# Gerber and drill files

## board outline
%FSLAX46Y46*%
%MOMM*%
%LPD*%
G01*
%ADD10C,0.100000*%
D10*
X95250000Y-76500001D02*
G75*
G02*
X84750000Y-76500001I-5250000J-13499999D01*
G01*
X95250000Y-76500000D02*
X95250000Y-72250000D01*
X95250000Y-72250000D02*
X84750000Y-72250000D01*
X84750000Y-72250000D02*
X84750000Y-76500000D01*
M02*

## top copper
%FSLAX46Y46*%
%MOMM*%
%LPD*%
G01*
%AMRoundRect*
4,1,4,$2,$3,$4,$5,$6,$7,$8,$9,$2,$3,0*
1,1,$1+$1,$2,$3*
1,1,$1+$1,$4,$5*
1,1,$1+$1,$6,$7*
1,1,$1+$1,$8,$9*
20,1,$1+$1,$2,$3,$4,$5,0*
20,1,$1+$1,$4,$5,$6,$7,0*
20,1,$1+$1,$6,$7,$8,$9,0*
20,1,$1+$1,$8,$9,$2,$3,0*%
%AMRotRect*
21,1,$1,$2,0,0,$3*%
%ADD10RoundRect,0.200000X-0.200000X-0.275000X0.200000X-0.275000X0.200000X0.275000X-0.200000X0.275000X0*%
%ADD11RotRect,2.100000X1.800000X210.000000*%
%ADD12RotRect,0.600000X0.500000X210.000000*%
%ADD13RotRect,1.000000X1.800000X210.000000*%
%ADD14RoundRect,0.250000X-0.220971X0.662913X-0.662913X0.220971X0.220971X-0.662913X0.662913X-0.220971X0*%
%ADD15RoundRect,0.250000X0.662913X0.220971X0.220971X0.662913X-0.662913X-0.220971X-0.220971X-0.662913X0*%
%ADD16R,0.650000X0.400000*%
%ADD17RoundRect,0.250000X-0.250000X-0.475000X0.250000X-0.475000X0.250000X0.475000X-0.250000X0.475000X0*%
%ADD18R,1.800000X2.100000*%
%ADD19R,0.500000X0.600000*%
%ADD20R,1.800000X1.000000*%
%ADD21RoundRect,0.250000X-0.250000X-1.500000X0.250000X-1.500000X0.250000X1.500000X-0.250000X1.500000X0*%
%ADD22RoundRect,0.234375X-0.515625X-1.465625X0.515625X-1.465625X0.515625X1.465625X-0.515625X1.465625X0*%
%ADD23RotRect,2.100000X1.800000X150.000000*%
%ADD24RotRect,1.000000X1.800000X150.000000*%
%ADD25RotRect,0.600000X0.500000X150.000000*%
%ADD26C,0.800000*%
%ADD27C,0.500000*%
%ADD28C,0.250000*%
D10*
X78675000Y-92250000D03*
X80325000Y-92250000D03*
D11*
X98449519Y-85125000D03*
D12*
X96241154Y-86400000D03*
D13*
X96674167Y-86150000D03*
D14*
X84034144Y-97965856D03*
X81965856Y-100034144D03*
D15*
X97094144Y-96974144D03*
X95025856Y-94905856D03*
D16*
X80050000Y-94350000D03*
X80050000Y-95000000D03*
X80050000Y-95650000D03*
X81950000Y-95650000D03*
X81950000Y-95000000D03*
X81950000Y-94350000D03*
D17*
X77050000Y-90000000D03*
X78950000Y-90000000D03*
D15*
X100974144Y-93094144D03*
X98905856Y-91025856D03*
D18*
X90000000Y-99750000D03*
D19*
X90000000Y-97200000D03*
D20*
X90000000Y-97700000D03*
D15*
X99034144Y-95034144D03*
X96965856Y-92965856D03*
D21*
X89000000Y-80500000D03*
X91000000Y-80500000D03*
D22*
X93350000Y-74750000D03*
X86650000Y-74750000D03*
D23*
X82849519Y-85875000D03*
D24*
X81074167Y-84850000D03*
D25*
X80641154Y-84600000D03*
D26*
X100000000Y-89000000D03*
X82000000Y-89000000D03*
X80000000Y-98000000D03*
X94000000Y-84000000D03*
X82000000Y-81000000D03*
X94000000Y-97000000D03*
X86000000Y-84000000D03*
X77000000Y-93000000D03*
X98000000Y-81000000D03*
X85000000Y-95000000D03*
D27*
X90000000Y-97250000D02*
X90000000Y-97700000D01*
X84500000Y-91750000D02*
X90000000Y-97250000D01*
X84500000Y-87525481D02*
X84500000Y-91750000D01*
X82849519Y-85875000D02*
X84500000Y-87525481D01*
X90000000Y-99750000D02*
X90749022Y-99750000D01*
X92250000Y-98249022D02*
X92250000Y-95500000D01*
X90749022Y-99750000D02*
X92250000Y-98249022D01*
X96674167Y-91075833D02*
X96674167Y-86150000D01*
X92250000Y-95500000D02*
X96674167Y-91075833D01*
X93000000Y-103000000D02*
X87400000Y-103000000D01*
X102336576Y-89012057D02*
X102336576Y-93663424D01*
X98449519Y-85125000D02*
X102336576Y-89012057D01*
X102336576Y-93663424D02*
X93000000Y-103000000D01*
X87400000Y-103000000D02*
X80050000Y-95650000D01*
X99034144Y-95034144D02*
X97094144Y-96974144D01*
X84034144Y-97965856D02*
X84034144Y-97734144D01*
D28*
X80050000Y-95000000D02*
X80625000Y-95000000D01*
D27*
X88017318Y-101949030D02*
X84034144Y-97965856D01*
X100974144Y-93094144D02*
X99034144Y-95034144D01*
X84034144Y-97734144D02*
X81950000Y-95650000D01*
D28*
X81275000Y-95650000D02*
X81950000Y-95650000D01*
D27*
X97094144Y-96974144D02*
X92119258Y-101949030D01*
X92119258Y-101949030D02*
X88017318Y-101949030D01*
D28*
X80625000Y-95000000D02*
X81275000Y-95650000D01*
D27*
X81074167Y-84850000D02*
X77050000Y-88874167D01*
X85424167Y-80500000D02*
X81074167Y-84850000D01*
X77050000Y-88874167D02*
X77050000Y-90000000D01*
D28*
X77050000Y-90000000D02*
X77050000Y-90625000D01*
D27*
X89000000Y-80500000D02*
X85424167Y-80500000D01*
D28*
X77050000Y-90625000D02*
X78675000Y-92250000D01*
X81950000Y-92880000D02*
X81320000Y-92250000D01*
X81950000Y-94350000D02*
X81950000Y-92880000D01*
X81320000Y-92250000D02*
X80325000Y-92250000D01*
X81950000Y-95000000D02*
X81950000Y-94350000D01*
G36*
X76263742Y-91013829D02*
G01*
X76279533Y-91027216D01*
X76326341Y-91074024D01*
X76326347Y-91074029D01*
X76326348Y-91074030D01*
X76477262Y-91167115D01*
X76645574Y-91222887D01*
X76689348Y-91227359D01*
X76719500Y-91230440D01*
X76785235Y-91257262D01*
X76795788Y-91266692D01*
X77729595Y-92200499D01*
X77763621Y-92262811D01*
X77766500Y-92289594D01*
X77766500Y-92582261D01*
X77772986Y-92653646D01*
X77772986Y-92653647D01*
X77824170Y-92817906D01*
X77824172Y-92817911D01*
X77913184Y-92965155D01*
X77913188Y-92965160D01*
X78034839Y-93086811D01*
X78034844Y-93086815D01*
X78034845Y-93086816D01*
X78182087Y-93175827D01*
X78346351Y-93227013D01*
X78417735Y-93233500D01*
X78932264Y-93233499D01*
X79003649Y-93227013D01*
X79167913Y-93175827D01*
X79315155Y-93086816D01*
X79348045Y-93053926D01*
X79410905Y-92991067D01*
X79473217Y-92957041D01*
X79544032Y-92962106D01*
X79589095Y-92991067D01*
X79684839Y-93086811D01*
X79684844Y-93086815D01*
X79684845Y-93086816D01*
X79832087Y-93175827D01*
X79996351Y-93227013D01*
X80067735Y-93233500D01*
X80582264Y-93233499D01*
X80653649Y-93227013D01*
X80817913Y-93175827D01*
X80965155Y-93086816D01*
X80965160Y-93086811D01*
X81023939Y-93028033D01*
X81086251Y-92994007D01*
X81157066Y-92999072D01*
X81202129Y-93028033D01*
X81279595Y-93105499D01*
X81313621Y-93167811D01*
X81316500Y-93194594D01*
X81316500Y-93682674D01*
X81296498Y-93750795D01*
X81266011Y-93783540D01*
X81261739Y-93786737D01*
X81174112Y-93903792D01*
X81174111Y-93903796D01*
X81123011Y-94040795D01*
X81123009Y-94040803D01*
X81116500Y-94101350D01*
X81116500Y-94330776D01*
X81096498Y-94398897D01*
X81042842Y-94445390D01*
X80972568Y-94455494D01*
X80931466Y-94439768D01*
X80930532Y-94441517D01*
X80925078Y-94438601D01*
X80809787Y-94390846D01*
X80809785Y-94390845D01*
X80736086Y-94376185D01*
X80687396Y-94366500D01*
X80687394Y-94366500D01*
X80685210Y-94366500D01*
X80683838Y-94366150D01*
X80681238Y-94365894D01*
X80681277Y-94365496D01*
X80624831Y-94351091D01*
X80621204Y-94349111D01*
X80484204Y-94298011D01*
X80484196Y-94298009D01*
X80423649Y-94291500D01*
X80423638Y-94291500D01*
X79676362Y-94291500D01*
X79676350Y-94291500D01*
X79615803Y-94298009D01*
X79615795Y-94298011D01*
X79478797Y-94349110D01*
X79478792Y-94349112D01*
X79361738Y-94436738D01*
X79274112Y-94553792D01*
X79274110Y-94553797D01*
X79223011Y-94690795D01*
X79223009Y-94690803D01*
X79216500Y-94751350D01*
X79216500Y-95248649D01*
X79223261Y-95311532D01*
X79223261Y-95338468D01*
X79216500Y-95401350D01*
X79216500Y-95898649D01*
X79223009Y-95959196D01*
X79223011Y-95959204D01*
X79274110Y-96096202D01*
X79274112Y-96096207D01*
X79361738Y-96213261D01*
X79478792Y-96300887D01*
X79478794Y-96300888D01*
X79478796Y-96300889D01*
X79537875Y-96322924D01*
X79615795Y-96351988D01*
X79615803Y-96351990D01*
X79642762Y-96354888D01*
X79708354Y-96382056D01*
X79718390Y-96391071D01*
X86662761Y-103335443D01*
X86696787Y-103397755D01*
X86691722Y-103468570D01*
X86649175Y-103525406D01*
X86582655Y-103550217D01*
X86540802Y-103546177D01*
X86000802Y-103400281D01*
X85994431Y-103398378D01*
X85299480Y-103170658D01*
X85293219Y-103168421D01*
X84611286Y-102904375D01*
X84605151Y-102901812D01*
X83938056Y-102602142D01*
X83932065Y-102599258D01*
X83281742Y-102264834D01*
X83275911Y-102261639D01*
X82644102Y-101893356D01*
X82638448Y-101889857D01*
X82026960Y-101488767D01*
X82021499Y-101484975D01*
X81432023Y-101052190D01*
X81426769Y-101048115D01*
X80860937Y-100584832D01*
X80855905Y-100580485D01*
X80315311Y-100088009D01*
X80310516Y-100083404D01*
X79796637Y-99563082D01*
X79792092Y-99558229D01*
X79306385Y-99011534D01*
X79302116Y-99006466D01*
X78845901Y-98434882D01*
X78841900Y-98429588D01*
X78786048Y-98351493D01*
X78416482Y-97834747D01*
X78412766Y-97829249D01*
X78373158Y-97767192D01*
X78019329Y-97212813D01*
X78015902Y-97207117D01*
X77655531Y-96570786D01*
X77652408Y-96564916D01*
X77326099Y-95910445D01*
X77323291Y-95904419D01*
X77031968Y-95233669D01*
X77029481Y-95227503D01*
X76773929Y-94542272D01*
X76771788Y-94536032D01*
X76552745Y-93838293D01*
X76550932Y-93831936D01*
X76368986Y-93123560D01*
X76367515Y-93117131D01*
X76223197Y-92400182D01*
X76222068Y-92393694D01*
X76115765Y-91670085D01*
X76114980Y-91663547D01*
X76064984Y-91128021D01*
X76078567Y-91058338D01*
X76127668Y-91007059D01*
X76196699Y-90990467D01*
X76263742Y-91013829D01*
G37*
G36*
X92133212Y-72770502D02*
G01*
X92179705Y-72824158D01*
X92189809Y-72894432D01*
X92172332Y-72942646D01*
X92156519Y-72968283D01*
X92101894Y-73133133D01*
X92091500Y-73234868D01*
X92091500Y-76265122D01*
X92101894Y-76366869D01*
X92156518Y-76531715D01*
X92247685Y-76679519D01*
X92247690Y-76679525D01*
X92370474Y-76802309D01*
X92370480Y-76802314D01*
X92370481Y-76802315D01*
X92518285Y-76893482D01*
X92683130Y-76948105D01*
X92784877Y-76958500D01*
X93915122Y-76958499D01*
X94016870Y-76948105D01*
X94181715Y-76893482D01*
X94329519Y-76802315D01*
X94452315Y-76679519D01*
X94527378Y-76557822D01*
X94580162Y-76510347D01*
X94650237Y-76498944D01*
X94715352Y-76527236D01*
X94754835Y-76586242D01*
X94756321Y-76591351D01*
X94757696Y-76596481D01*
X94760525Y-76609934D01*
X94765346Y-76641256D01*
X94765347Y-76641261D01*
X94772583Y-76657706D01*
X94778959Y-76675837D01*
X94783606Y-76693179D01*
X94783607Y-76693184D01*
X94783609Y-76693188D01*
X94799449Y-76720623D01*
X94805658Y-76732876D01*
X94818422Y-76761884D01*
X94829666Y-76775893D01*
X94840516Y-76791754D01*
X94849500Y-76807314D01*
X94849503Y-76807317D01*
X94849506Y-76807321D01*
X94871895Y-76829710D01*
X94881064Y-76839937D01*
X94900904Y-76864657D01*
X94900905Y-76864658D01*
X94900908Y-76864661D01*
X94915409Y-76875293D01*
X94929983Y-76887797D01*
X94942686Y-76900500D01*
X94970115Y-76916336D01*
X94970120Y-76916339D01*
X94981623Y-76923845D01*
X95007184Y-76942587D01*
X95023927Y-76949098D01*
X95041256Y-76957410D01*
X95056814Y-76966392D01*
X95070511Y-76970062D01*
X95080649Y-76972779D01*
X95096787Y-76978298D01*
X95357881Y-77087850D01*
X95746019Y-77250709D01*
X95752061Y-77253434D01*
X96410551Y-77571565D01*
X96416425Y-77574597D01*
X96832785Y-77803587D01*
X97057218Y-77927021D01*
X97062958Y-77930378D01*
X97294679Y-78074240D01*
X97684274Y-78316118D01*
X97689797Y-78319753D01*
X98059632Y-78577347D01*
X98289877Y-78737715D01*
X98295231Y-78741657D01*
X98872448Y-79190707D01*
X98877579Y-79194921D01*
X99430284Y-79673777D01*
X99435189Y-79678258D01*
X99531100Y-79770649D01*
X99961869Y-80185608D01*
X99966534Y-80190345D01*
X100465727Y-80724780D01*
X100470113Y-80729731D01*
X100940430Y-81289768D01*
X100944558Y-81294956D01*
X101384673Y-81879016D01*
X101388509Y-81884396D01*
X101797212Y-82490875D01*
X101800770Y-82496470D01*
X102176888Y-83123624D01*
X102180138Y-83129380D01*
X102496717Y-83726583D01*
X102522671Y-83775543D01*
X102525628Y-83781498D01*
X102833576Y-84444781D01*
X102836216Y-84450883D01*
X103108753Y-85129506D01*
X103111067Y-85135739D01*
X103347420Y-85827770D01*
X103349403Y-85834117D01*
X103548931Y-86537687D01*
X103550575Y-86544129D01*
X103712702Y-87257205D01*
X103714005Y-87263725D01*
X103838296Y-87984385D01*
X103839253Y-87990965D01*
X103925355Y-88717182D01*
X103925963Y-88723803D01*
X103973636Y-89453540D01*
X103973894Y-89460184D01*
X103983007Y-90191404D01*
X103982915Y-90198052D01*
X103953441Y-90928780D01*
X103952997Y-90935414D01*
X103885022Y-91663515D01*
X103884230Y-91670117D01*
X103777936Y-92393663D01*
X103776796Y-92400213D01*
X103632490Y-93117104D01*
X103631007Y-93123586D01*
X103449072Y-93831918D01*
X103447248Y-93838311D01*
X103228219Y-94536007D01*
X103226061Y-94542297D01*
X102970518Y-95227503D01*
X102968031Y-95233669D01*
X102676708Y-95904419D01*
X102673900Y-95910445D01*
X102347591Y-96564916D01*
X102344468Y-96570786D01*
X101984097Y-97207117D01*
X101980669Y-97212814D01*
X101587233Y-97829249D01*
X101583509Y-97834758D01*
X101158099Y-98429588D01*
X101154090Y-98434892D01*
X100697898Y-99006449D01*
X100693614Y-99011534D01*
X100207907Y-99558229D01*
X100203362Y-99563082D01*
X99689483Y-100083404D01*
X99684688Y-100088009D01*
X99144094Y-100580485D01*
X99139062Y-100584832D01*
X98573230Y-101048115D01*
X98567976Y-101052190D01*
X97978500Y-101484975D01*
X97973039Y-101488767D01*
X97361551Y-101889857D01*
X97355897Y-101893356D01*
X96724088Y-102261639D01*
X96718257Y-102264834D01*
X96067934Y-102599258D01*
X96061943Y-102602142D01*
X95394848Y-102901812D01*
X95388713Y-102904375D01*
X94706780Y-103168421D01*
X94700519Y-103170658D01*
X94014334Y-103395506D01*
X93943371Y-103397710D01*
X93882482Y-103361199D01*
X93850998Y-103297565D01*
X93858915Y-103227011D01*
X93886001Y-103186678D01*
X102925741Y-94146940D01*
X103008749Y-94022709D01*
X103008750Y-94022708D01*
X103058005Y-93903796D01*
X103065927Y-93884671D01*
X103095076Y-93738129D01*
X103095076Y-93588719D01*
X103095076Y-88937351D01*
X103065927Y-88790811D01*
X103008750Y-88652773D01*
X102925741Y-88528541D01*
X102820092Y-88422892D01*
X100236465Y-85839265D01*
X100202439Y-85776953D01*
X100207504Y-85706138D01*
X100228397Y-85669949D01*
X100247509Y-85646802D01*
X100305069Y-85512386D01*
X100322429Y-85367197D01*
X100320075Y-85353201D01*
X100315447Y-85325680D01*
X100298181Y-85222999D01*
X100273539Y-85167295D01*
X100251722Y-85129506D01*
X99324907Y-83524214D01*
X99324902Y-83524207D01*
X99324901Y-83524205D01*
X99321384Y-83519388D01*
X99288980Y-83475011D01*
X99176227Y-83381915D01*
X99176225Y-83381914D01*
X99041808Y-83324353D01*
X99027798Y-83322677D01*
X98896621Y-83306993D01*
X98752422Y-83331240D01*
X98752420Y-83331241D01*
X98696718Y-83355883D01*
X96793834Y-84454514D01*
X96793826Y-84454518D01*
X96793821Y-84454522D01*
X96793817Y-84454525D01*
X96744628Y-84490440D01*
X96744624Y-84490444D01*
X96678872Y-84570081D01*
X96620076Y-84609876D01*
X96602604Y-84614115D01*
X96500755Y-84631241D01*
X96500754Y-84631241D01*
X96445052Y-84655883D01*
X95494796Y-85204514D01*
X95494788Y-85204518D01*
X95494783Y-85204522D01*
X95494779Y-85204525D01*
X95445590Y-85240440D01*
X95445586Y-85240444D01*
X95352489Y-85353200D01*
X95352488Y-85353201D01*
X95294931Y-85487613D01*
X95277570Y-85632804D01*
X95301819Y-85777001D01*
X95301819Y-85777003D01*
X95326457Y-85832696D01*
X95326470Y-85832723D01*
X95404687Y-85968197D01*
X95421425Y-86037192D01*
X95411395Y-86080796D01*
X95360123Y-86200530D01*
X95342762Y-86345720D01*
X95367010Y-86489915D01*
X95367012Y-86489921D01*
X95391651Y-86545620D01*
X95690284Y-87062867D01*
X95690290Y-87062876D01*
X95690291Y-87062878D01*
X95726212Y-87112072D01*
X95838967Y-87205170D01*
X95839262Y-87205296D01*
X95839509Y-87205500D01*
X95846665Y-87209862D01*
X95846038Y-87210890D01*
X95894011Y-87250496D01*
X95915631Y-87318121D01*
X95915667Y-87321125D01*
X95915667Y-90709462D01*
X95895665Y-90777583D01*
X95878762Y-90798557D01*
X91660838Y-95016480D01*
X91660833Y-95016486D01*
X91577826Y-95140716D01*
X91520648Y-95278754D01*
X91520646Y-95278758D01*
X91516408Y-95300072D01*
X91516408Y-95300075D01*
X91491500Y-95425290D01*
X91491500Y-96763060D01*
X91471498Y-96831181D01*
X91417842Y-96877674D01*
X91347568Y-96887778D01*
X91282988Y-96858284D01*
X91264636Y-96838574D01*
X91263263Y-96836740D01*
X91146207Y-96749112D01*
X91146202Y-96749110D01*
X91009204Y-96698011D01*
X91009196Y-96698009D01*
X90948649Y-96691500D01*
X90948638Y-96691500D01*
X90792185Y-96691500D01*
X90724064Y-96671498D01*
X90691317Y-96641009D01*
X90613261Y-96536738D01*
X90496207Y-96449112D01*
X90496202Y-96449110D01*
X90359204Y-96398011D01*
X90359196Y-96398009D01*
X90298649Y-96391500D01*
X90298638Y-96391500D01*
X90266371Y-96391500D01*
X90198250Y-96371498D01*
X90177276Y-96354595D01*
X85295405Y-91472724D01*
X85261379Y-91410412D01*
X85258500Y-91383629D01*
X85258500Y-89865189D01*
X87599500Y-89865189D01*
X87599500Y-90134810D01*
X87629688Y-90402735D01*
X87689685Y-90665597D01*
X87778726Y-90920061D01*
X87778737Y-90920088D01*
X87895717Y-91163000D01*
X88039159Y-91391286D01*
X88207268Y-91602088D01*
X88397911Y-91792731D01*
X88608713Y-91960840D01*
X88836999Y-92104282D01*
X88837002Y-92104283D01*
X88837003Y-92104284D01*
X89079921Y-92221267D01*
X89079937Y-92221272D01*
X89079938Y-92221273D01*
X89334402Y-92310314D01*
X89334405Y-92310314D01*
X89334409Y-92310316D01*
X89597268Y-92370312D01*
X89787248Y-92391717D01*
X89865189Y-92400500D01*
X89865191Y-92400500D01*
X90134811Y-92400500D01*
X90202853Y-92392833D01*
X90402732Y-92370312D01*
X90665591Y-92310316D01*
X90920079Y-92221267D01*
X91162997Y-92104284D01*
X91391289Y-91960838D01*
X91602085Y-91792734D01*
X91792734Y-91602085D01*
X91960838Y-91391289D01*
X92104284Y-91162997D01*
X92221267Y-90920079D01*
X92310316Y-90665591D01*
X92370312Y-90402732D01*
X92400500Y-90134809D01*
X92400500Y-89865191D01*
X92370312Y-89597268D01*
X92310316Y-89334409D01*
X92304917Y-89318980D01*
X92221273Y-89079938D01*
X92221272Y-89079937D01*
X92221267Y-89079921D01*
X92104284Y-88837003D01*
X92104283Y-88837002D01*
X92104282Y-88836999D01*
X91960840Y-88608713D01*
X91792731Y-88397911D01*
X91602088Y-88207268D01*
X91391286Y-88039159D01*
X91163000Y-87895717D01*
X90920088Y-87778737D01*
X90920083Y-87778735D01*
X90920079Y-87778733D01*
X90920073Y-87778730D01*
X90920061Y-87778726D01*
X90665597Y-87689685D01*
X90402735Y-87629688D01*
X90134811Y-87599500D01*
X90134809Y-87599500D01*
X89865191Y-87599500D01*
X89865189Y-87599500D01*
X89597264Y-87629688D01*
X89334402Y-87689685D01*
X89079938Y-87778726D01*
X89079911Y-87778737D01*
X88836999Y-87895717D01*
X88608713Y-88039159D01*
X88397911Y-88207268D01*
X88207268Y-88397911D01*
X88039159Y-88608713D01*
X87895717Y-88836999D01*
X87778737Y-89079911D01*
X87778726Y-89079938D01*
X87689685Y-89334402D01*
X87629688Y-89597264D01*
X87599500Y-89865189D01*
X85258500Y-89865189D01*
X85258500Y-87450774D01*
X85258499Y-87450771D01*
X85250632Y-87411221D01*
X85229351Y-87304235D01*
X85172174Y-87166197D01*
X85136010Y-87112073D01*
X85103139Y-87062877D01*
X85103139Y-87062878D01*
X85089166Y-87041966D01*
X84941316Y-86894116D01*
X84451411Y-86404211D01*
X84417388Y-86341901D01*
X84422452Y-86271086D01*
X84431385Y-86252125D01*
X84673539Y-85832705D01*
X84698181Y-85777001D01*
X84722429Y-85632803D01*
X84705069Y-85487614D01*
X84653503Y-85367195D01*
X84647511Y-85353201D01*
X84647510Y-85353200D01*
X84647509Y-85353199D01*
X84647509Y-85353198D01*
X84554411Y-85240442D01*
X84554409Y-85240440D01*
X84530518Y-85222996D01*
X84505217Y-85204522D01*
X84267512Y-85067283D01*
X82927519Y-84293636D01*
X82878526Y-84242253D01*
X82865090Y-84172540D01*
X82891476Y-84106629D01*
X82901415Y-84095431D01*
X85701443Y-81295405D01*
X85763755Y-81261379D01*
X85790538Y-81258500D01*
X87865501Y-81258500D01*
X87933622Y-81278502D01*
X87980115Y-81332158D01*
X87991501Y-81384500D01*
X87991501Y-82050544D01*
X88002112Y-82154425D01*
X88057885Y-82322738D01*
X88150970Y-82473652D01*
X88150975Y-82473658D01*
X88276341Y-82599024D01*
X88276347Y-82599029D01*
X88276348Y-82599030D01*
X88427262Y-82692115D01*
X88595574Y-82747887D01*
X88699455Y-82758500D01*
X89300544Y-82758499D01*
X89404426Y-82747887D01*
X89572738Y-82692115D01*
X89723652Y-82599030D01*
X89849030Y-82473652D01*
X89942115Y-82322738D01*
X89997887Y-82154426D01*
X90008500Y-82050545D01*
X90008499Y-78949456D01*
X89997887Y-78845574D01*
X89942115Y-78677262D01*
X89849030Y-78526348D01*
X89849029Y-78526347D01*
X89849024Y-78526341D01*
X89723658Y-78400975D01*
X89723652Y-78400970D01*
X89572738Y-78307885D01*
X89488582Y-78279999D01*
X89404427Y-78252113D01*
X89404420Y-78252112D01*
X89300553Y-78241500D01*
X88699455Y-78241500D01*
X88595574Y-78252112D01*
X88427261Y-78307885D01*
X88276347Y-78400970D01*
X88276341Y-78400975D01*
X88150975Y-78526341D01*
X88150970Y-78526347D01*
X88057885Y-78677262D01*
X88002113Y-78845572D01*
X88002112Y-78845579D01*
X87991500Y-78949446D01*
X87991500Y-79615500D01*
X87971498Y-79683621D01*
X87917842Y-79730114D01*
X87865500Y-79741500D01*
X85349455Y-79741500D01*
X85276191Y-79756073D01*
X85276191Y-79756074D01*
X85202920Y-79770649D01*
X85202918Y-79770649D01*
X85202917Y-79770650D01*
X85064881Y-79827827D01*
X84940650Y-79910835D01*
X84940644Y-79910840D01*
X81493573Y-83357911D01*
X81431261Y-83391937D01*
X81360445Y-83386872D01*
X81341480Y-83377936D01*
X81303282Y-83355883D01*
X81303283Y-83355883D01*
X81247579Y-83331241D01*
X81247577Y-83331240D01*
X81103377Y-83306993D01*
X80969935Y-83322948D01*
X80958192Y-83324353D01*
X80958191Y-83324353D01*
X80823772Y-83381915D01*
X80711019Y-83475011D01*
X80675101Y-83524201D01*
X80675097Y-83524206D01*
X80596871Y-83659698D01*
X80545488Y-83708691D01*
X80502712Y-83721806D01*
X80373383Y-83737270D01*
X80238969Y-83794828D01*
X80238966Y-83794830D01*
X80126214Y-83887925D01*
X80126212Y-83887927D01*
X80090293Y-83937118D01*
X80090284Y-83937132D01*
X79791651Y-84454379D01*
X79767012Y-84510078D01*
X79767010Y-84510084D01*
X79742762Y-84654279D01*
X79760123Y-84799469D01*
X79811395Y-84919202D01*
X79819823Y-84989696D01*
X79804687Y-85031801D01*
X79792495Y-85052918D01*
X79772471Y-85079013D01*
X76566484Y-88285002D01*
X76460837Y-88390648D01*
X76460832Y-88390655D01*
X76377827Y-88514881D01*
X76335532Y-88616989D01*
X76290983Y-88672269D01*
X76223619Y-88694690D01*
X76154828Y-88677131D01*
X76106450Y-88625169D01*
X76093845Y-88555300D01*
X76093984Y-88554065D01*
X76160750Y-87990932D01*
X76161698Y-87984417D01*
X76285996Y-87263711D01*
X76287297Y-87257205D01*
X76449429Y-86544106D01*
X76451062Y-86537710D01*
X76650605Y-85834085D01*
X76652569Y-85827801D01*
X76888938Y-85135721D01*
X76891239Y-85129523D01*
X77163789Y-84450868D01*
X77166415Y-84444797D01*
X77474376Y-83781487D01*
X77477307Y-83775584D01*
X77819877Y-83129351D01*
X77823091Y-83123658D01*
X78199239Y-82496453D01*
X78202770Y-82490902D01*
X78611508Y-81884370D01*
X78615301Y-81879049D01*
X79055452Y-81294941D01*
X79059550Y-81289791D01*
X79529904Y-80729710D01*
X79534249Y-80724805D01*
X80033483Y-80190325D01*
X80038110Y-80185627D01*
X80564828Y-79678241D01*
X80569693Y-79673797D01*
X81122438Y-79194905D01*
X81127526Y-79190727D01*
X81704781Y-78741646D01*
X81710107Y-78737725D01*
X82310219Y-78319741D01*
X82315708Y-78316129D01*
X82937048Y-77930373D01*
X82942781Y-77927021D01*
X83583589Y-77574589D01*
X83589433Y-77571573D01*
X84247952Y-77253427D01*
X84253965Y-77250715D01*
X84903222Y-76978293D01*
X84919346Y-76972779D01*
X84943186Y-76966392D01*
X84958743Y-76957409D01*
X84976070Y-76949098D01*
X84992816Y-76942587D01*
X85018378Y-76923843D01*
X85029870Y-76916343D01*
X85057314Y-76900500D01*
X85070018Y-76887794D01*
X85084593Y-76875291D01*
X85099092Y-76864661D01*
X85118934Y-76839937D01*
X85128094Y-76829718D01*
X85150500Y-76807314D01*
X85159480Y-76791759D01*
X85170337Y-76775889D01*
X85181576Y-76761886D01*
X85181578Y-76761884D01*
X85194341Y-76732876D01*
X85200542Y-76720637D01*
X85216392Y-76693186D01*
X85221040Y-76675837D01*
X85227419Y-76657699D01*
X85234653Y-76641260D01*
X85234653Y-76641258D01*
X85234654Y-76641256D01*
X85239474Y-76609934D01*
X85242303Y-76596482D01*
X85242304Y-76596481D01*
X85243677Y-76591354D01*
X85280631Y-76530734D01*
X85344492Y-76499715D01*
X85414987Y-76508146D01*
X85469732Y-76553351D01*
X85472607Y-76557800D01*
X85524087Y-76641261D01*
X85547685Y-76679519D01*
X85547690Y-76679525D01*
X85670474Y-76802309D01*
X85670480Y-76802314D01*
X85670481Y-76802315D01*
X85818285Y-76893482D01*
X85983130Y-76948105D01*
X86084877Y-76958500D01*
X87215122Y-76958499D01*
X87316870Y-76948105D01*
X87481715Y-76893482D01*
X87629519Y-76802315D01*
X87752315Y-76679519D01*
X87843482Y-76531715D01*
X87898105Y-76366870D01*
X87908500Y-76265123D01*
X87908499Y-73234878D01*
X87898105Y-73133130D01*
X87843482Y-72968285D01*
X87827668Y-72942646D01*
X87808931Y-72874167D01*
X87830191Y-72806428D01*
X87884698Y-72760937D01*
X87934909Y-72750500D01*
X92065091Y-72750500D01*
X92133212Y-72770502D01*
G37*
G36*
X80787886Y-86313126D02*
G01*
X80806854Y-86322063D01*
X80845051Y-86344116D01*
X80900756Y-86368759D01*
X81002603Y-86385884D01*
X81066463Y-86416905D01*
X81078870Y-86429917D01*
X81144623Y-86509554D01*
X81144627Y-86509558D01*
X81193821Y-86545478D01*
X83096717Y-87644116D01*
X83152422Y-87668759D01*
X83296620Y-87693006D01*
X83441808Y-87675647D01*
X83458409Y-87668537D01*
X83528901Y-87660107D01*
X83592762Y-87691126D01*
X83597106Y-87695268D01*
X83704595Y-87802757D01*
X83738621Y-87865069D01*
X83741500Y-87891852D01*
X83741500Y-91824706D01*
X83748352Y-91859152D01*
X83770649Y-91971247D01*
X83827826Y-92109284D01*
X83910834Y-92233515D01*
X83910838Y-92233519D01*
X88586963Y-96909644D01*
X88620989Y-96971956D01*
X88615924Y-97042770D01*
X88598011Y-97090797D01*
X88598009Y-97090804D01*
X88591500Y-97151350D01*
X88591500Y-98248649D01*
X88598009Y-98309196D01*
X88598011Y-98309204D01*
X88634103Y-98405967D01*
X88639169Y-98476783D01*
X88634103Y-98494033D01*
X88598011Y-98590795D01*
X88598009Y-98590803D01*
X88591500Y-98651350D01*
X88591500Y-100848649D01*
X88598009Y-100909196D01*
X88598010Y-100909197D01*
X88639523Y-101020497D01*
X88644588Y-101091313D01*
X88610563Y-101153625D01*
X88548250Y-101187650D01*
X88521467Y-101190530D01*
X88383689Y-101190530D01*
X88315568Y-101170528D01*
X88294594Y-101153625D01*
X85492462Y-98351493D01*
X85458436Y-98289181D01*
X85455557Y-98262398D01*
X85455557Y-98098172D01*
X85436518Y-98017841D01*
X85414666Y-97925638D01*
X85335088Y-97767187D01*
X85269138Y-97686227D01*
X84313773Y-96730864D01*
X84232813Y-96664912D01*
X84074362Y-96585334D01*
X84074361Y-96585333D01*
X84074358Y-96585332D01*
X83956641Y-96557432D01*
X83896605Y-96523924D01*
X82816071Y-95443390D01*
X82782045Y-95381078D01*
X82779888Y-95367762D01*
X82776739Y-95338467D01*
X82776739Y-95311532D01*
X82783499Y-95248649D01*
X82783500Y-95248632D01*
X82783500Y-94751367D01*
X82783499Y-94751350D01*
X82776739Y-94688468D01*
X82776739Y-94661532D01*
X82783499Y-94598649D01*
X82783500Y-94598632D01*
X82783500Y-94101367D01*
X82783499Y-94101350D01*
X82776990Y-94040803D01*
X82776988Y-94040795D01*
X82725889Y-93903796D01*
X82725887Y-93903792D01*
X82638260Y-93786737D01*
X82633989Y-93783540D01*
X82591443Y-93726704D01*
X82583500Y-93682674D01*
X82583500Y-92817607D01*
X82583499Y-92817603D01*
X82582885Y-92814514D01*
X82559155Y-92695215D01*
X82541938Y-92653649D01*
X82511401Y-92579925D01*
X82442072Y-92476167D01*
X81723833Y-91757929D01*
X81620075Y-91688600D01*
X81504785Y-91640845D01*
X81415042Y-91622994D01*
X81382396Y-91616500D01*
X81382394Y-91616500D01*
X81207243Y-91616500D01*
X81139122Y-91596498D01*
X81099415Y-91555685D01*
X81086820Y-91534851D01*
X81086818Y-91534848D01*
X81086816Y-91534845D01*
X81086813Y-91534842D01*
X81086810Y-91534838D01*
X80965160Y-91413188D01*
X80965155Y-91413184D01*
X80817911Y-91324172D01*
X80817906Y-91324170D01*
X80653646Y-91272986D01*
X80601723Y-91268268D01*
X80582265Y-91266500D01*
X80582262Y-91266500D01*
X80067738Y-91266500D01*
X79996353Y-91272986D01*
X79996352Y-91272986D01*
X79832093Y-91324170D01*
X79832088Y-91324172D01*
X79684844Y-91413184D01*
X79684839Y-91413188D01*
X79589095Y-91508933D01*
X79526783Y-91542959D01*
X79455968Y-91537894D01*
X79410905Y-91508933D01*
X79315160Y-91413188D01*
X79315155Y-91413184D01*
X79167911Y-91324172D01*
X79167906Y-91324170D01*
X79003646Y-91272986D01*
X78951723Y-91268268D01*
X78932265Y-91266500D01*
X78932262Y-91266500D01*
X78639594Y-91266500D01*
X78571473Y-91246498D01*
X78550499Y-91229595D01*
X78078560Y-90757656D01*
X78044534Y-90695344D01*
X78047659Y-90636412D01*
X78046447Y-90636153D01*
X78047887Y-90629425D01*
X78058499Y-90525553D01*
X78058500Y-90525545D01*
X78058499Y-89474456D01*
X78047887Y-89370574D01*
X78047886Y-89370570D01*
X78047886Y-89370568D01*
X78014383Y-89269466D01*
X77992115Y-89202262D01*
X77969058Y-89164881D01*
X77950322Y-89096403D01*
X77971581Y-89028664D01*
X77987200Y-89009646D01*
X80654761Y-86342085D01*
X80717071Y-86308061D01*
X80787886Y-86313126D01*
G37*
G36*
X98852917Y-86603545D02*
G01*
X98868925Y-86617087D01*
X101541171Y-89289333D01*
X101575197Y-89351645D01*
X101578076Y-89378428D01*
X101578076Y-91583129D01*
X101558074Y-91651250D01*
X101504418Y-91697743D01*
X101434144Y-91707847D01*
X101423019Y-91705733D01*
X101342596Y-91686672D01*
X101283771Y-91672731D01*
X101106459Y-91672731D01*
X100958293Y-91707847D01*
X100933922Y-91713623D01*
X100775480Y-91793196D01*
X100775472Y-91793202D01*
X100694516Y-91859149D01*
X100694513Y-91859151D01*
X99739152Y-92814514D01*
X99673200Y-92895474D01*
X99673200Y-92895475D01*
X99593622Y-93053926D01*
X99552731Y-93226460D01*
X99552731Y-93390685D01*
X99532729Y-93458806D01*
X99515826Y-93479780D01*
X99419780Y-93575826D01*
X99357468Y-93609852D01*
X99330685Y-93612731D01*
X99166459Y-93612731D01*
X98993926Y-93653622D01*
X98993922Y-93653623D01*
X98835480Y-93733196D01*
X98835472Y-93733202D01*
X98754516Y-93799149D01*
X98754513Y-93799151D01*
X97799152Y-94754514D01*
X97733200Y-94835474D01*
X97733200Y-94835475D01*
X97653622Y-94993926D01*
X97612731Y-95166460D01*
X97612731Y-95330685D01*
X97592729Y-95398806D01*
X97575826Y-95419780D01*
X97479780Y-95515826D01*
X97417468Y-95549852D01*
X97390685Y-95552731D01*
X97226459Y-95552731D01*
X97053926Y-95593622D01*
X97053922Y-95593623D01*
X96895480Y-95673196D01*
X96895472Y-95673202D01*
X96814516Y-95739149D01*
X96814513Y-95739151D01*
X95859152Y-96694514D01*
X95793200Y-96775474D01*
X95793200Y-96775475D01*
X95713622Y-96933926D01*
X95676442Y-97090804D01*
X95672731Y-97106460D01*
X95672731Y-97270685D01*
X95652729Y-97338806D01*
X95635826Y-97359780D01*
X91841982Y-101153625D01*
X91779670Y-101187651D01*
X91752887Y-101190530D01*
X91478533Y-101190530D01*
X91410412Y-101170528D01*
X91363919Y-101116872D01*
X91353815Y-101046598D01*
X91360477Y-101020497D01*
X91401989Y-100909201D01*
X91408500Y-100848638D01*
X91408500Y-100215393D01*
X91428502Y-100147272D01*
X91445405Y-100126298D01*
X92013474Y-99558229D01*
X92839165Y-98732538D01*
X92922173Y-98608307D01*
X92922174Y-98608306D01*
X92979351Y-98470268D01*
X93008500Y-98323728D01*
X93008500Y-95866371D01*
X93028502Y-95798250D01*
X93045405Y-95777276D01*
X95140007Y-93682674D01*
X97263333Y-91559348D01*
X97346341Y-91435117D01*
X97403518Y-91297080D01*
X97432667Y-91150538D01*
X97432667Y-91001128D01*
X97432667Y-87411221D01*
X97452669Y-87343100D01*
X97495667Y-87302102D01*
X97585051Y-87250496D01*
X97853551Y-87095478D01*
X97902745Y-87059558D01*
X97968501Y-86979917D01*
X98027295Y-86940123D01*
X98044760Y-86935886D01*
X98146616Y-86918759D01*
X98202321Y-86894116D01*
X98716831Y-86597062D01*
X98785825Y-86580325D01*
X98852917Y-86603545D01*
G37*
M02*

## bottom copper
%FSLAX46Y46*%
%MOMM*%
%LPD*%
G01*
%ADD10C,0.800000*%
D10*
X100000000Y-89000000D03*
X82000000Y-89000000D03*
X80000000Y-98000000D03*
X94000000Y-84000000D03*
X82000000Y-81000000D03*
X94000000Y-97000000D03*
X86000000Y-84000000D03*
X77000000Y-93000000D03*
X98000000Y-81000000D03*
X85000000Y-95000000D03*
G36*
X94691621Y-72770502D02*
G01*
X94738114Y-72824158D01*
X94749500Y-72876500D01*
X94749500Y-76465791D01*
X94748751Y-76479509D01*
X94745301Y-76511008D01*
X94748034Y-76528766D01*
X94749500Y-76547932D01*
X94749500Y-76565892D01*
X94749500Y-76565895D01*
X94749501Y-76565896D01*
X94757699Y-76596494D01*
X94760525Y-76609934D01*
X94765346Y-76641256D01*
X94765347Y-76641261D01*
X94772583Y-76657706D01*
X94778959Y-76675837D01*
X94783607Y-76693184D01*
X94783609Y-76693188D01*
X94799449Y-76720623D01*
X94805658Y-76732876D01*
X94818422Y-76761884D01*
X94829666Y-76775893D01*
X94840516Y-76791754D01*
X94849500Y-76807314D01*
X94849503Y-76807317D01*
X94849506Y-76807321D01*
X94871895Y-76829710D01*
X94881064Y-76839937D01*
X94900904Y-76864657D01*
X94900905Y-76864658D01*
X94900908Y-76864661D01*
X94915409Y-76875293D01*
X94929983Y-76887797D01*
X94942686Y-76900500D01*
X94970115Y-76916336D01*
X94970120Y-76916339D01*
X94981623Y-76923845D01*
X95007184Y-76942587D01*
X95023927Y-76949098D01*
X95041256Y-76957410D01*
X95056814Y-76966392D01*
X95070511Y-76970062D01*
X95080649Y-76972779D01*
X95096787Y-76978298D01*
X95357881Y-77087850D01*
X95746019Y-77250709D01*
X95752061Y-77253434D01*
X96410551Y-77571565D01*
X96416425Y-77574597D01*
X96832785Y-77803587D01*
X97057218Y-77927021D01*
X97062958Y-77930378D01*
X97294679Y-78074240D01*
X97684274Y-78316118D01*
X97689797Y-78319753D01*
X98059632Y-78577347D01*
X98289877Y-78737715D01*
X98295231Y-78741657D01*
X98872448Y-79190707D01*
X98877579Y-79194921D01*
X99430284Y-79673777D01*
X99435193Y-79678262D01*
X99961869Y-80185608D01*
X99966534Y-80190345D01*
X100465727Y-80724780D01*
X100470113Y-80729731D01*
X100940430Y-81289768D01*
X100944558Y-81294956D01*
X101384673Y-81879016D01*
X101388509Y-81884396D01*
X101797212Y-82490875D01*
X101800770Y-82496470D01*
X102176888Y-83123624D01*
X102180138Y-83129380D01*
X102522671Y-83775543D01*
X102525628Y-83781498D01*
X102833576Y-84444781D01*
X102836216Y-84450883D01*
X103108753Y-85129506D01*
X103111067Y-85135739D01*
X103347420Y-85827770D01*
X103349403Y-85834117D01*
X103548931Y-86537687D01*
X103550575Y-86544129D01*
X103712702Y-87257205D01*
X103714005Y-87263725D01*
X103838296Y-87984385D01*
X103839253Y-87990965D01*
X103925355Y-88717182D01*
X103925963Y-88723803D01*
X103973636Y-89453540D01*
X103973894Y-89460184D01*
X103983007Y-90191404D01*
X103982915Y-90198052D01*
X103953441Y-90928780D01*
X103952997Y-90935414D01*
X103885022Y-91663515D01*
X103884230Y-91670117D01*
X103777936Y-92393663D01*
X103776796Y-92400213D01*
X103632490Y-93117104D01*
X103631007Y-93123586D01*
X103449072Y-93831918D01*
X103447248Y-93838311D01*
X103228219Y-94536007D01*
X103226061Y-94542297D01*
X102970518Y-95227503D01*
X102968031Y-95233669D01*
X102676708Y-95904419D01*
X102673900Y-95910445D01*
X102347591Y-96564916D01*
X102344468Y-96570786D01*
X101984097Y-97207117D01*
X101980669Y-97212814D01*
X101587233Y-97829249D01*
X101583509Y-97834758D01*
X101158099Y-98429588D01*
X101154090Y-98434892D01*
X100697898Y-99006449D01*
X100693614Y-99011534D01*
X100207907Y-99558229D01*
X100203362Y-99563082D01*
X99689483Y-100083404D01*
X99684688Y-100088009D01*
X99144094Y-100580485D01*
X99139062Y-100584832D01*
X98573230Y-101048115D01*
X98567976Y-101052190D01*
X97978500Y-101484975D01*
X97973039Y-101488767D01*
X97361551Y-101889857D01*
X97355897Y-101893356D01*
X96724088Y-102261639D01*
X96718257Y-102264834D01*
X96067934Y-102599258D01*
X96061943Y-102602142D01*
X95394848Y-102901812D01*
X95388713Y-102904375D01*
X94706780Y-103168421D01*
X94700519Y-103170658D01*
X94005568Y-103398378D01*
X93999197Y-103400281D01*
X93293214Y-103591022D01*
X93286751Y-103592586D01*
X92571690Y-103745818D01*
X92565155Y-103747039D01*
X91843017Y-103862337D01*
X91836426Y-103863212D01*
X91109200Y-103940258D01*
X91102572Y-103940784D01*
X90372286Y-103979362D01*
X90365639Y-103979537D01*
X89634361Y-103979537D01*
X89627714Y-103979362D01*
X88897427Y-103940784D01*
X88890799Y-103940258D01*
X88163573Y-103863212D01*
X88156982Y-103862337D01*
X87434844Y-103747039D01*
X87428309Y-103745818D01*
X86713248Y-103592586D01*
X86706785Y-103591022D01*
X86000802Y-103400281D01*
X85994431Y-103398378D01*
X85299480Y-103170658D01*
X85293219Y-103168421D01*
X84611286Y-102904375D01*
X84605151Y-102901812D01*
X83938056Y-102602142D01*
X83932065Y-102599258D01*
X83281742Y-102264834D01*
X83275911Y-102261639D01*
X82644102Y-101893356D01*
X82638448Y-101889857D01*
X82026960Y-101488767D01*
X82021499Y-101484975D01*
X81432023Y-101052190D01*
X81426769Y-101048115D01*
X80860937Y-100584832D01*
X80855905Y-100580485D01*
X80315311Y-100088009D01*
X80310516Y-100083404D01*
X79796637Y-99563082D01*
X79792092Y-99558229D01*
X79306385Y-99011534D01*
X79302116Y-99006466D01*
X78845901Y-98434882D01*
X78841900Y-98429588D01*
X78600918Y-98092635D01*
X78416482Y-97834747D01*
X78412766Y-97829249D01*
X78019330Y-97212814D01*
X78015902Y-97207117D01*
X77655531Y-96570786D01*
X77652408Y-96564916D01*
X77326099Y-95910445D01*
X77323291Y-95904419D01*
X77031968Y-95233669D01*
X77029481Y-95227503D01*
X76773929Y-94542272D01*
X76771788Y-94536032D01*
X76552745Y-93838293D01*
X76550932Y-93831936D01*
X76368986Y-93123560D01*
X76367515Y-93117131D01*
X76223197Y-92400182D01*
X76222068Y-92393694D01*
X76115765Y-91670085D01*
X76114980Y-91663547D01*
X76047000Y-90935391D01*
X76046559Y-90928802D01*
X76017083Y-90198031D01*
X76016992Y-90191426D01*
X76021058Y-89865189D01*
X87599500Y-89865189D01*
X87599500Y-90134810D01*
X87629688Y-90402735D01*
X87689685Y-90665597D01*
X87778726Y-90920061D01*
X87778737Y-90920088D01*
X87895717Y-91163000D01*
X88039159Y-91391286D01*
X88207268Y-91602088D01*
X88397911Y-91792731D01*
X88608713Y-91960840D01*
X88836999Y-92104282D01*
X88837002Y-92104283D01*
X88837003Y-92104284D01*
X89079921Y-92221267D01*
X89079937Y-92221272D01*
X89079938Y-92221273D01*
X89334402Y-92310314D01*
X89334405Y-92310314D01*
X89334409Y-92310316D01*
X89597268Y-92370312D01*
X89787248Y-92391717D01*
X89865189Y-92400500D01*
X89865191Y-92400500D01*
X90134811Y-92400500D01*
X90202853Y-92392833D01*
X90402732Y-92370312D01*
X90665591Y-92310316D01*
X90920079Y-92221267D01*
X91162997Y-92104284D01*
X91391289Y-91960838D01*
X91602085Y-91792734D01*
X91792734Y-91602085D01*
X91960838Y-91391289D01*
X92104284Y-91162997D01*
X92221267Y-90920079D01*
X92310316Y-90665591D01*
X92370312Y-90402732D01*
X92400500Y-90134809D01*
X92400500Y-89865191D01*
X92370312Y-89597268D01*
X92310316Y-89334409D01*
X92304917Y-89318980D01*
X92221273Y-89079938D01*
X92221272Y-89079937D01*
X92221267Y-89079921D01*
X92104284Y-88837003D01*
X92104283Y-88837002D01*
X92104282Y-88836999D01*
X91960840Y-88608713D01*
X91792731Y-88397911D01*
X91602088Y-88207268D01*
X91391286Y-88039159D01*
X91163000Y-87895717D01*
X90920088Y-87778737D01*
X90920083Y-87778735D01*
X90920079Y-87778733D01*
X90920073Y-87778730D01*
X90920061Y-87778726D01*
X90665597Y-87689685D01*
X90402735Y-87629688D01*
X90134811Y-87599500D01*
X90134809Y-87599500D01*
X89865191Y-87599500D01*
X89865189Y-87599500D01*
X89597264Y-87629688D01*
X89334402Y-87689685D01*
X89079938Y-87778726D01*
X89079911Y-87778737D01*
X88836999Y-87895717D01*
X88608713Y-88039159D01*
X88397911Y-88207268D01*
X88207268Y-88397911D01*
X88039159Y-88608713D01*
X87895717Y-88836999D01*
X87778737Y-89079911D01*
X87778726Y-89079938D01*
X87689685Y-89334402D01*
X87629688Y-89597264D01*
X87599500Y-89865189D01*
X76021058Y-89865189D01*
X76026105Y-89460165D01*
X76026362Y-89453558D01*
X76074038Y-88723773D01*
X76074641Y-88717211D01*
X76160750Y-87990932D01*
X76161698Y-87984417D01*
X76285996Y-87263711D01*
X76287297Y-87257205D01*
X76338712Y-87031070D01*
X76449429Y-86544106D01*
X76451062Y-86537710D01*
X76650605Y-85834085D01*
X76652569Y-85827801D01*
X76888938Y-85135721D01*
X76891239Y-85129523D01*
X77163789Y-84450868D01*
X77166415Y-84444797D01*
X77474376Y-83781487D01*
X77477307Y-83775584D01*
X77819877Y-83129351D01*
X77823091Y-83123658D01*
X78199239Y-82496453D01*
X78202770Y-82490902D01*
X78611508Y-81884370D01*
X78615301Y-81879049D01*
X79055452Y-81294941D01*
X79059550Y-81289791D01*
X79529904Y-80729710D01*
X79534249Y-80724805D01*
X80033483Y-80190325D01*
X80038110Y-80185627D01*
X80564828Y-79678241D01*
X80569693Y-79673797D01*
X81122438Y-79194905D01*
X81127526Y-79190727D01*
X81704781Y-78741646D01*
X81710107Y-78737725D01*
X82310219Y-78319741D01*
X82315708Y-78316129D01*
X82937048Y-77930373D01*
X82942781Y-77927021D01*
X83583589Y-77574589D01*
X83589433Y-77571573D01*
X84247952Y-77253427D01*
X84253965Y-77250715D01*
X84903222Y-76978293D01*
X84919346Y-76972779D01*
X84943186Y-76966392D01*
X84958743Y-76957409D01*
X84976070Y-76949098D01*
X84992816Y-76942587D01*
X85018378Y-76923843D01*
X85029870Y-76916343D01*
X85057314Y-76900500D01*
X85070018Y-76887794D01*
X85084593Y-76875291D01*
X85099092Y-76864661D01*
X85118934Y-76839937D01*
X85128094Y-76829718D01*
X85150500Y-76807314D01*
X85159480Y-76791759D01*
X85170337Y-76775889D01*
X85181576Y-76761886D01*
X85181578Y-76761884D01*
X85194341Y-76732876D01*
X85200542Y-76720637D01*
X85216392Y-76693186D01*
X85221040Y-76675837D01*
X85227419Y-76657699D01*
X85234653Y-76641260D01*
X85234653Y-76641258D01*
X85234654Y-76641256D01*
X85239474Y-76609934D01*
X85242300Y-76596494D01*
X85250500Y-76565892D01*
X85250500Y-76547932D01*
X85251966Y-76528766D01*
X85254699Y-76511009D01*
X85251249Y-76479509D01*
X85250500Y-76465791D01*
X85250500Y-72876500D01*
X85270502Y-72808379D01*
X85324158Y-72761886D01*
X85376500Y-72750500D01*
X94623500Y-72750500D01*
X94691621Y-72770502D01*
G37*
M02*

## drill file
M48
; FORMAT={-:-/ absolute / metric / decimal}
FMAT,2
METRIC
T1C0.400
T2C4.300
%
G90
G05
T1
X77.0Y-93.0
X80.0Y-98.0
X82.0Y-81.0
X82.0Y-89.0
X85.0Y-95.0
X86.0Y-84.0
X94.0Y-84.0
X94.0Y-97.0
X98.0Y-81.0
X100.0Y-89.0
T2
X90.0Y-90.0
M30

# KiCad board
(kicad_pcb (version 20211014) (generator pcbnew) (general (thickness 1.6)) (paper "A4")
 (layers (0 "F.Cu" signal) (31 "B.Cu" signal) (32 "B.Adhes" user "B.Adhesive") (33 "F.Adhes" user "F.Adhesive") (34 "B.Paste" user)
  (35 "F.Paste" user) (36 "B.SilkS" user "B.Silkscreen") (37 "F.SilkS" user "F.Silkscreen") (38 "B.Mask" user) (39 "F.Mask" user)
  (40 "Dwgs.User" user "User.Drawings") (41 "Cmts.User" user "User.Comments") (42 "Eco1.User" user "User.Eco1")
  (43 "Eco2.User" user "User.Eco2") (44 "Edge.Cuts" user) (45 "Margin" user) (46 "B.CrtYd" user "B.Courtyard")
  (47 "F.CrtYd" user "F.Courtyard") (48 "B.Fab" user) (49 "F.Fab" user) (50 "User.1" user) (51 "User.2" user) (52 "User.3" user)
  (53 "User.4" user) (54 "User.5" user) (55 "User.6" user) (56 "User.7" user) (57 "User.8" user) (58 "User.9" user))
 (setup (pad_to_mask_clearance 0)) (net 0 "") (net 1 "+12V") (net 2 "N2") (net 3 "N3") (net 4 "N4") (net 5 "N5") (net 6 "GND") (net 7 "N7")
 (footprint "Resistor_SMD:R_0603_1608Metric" (layer "F.Cu") (at 79.5 92.25)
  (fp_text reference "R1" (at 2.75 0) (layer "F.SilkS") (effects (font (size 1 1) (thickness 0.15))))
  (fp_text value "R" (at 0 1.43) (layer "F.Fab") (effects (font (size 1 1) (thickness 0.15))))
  (pad "1" smd roundrect (at -0.825 0) (size 0.8 0.95) (layers "F.Cu" "F.Paste" "F.Mask") (roundrect_rratio 0.25) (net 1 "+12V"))
  (pad "2" smd roundrect (at 0.825 0) (size 0.8 0.95) (layers "F.Cu" "F.Paste" "F.Mask") (roundrect_rratio 0.25) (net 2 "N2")))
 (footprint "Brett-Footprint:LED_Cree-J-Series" (layer "F.Cu") (at 97.8 85.5 -150)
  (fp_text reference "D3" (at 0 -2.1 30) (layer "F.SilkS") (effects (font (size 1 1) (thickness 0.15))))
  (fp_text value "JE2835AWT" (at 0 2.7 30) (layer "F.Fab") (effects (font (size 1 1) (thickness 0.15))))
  (pad "" smd rect (at -0.75 0 210) (size 1.7 1.5) (layers "F.Paste"))
  (pad "" smd rect (at 1.3 0 210) (size 0.8 1.5) (layers "F.Paste"))
  (pad "1" smd rect (at -0.75 0 210) (size 2.1 1.8) (layers "F.Cu" "F.Mask") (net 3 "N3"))
  (pad "2" smd rect (at 1.8 0 210) (size 0.6 0.5) (layers "F.Cu" "F.Mask") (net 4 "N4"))
  (pad "2" smd rect (at 1.3 0 210) (size 1 1.8) (layers "F.Cu" "F.Mask") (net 4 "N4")))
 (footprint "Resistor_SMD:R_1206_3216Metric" (layer "F.Cu") (at 83 99 -135)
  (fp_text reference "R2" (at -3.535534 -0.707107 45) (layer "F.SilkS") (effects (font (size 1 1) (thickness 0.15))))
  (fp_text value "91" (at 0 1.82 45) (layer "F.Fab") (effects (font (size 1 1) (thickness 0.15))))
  (pad "1" smd roundrect (at -1.4625 0 225) (size 1.125 1.75) (layers "F.Cu" "F.Paste" "F.Mask") (roundrect_rratio 0.2222222222)
   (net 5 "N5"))
  (pad "2" smd roundrect (at 1.4625 0 225) (size 1.125 1.75) (layers "F.Cu" "F.Paste" "F.Mask") (roundrect_rratio 0.2222222222)
   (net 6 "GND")))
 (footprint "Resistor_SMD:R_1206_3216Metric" (layer "F.Cu") (at 96.06 95.94 135)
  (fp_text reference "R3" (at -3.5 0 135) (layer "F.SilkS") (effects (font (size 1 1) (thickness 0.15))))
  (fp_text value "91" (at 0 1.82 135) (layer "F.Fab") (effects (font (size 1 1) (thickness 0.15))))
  (pad "1" smd roundrect (at -1.4625 0 135) (size 1.125 1.75) (layers "F.Cu" "F.Paste" "F.Mask") (roundrect_rratio 0.2222222222)
   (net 5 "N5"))
  (pad "2" smd roundrect (at 1.4625 0 135) (size 1.125 1.75) (layers "F.Cu" "F.Paste" "F.Mask") (roundrect_rratio 0.2222222222)
   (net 6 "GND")))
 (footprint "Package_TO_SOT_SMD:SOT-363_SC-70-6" (layer "F.Cu") (at 81 95)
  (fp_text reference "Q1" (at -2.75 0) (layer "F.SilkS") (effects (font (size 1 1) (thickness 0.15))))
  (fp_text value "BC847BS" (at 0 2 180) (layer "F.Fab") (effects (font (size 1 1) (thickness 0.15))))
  (pad "1" smd rect (at -0.95 -0.65) (size 0.65 0.4) (layers "F.Cu" "F.Paste" "F.Mask") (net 6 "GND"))
  (pad "2" smd rect (at -0.95 0) (size 0.65 0.4) (layers "F.Cu" "F.Paste" "F.Mask") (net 5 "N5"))
  (pad "3" smd rect (at -0.95 0.65) (size 0.65 0.4) (layers "F.Cu" "F.Paste" "F.Mask") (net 3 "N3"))
  (pad "4" smd rect (at 0.95 0.65) (size 0.65 0.4) (layers "F.Cu" "F.Paste" "F.Mask") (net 5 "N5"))
  (pad "5" smd rect (at 0.95 0) (size 0.65 0.4) (layers "F.Cu" "F.Paste" "F.Mask") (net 2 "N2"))
  (pad "6" smd rect (at 0.95 -0.65) (size 0.65 0.4) (layers "F.Cu" "F.Paste" "F.Mask") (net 2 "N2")))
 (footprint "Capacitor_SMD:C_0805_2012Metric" (layer "F.Cu") (at 78 90)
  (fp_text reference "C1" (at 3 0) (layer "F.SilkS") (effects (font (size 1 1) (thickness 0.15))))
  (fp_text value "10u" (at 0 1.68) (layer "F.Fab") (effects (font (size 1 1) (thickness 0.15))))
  (pad "1" smd roundrect (at -0.95 0) (size 1 1.45) (layers "F.Cu" "F.Paste" "F.Mask") (roundrect_rratio 0.25) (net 1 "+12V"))
  (pad "2" smd roundrect (at 0.95 0) (size 1 1.45) (layers "F.Cu" "F.Paste" "F.Mask") (roundrect_rratio 0.25) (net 6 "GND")))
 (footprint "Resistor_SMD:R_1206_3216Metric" (layer "F.Cu") (at 99.94 92.06 135)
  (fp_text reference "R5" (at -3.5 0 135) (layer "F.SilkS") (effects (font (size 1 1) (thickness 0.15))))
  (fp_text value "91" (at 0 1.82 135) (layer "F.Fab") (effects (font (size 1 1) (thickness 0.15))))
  (pad "1" smd roundrect (at -1.4625 0 135) (size 1.125 1.75) (layers "F.Cu" "F.Paste" "F.Mask") (roundrect_rratio 0.2222222222)
   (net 5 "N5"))
  (pad "2" smd roundrect (at 1.4625 0 135) (size 1.125 1.75) (layers "F.Cu" "F.Paste" "F.Mask") (roundrect_rratio 0.2222222222)
   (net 6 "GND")))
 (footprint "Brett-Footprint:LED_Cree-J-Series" (layer "F.Cu") (at 90 99 90)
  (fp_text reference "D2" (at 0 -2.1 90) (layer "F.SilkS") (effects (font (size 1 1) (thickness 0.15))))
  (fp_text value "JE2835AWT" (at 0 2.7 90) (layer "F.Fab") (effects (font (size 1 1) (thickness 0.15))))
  (pad "" smd rect (at 1.3 0 90) (size 0.8 1.5) (layers "F.Paste"))
  (pad "" smd rect (at -0.75 0 90) (size 1.7 1.5) (layers "F.Paste"))
  (pad "1" smd rect (at -0.75 0 90) (size 2.1 1.8) (layers "F.Cu" "F.Mask") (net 4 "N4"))
  (pad "2" smd rect (at 1.8 0 90) (size 0.6 0.5) (layers "F.Cu" "F.Mask") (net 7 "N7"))
  (pad "2" smd rect (at 1.3 0 90) (size 1 1.8) (layers "F.Cu" "F.Mask") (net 7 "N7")))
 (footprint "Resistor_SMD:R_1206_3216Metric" (layer "F.Cu") (at 98 94 135)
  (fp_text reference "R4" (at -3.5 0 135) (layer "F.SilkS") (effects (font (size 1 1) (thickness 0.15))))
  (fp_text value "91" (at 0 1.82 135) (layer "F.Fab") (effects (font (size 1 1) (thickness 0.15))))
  (pad "1" smd roundrect (at -1.4625 0 135) (size 1.125 1.75) (layers "F.Cu" "F.Paste" "F.Mask") (roundrect_rratio 0.2222222222)
   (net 5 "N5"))
  (pad "2" smd roundrect (at 1.4625 0 135) (size 1.125 1.75) (layers "F.Cu" "F.Paste" "F.Mask") (roundrect_rratio 0.2222222222)
   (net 6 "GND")))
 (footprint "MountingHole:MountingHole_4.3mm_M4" (layer "F.Cu") (at 90 90)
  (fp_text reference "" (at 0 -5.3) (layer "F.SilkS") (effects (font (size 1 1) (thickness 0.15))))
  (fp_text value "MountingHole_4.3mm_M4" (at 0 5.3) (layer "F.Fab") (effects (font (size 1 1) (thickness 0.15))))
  (pad "" np_thru_hole circle (at 0 0) (size 4.3 4.3) (drill 4.3) (layers *.Cu *.Mask)))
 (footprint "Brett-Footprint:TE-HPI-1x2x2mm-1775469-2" (layer "F.Cu") (at 90 78)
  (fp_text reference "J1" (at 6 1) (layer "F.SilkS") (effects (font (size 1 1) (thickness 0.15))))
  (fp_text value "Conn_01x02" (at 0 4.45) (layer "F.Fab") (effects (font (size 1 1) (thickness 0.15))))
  (pad "1" smd roundrect (at -1 2.5) (size 1 3.5) (layers "F.Cu" "F.Paste" "F.Mask") (roundrect_rratio 0.25) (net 1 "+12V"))
  (pad "2" smd roundrect (at 1 2.5) (size 1 3.5) (layers "F.Cu" "F.Paste" "F.Mask") (roundrect_rratio 0.25) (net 6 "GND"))
  (pad "MP" smd roundrect (at 3.35 -3.25) (size 1.5 3.4) (layers "F.Cu" "F.Paste" "F.Mask") (roundrect_rratio 0.15625))
  (pad "MP" smd roundrect (at -3.35 -3.25) (size 1.5 3.4) (layers "F.Cu" "F.Paste" "F.Mask") (roundrect_rratio 0.15625)))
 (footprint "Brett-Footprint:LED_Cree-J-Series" (layer "F.Cu") (at 82.2 85.5 150)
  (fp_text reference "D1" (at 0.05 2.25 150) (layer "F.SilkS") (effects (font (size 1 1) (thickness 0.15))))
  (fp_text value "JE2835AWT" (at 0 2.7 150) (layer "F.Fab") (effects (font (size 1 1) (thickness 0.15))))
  (pad "" smd rect (at 1.3 0 150) (size 0.8 1.5) (layers "F.Paste"))
  (pad "" smd rect (at -0.75 0 150) (size 1.7 1.5) (layers "F.Paste"))
  (pad "1" smd rect (at -0.75 0 150) (size 2.1 1.8) (layers "F.Cu" "F.Mask") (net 7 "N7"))
  (pad "2" smd rect (at 1.3 0 150) (size 1 1.8) (layers "F.Cu" "F.Mask") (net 1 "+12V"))
  (pad "2" smd rect (at 1.8 0 150) (size 0.6 0.5) (layers "F.Cu" "F.Mask") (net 1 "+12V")))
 (gr_arc (start 95.25 76.500001) (mid 90 104.484905) (end 84.75 76.500001) (layer "Edge.Cuts") (width 0.1))
 (gr_line (start 95.25 76.5) (end 95.25 72.25) (layer "Edge.Cuts") (width 0.1))
 (gr_line (start 95.25 72.25) (end 84.75 72.25) (layer "Edge.Cuts") (width 0.1))
 (gr_line (start 84.75 72.25) (end 84.75 76.5) (layer "Edge.Cuts") (width 0.1))
 (segment (start 90 97.25) (end 90 97.7) (width 0.5) (layer "F.Cu") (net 7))
 (segment (start 84.5 91.75) (end 90 97.25) (width 0.5) (layer "F.Cu") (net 7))
 (segment (start 84.5 87.525481) (end 84.5 91.75) (width 0.5) (layer "F.Cu") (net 7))
 (segment (start 82.849519 85.875) (end 84.5 87.525481) (width 0.5) (layer "F.Cu") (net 7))
 (segment (start 90 99.75) (end 90.749022 99.75) (width 0.5) (layer "F.Cu") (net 4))
 (segment (start 92.25 98.249022) (end 92.25 95.5) (width 0.5) (layer "F.Cu") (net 4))
 (segment (start 90.749022 99.75) (end 92.25 98.249022) (width 0.5) (layer "F.Cu") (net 4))
 (segment (start 96.674167 91.075833) (end 96.674167 86.15) (width 0.5) (layer "F.Cu") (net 4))
 (segment (start 92.25 95.5) (end 96.674167 91.075833) (width 0.5) (layer "F.Cu") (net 4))
 (segment (start 93 103) (end 87.4 103) (width 0.5) (layer "F.Cu") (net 3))
 (segment (start 102.336576 89.012057) (end 102.336576 93.663424) (width 0.5) (layer "F.Cu") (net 3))
 (segment (start 98.449519 85.125) (end 102.336576 89.012057) (width 0.5) (layer "F.Cu") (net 3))
 (segment (start 102.336576 93.663424) (end 93 103) (width 0.5) (layer "F.Cu") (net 3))
 (segment (start 87.4 103) (end 80.05 95.65) (width 0.5) (layer "F.Cu") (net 3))
 (segment (start 99.034144 95.034144) (end 97.094144 96.974144) (width 0.5) (layer "F.Cu") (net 5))
 (segment (start 84.034144 97.965856) (end 84.034144 97.734144) (width 0.5) (layer "F.Cu") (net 5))
 (segment (start 80.05 95) (end 80.625 95) (width 0.25) (layer "F.Cu") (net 5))
 (segment (start 88.017318 101.94903) (end 84.034144 97.965856) (width 0.5) (layer "F.Cu") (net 5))
 (segment (start 100.974144 93.094144) (end 99.034144 95.034144) (width 0.5) (layer "F.Cu") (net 5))
 (segment (start 84.034144 97.734144) (end 81.95 95.65) (width 0.5) (layer "F.Cu") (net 5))
 (segment (start 81.275 95.65) (end 81.95 95.65) (width 0.25) (layer "F.Cu") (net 5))
 (segment (start 97.094144 96.974144) (end 92.119258 101.94903) (width 0.5) (layer "F.Cu") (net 5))
 (segment (start 92.119258 101.94903) (end 88.017318 101.94903) (width 0.5) (layer "F.Cu") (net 5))
 (segment (start 80.625 95) (end 81.275 95.65) (width 0.25) (layer "F.Cu") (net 5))
 (segment (start 81.074167 84.85) (end 77.05 88.874167) (width 0.5) (layer "F.Cu") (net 1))
 (segment (start 85.424167 80.5) (end 81.074167 84.85) (width 0.5) (layer "F.Cu") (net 1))
 (segment (start 77.05 88.874167) (end 77.05 90) (width 0.5) (layer "F.Cu") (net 1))
 (segment (start 77.05 90) (end 77.05 90.625) (width 0.25) (layer "F.Cu") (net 1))
 (segment (start 89 80.5) (end 85.424167 80.5) (width 0.5) (layer "F.Cu") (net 1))
 (segment (start 77.05 90.625) (end 78.675 92.25) (width 0.25) (layer "F.Cu") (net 1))
 (via (at 100 89) (size 0.8) (drill 0.4) (layers "F.Cu" "B.Cu") (free) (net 6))
 (via (at 82 89) (size 0.8) (drill 0.4) (layers "F.Cu" "B.Cu") (free) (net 6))
 (via (at 80 98) (size 0.8) (drill 0.4) (layers "F.Cu" "B.Cu") (free) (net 6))
 (via (at 94 84) (size 0.8) (drill 0.4) (layers "F.Cu" "B.Cu") (free) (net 6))
 (via (at 82 81) (size 0.8) (drill 0.4) (layers "F.Cu" "B.Cu") (free) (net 6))
 (via (at 94 97) (size 0.8) (drill 0.4) (layers "F.Cu" "B.Cu") (free) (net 6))
 (via (at 86 84) (size 0.8) (drill 0.4) (layers "F.Cu" "B.Cu") (free) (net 6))
 (via (at 77 93) (size 0.8) (drill 0.4) (layers "F.Cu" "B.Cu") (free) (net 6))
 (via (at 98 81) (size 0.8) (drill 0.4) (layers "F.Cu" "B.Cu") (free) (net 6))
 (via (at 85 95) (size 0.8) (drill 0.4) (layers "F.Cu" "B.Cu") (free) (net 6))
 (segment (start 81.95 92.88) (end 81.32 92.25) (width 0.25) (layer "F.Cu") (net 2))
 (segment (start 81.95 94.35) (end 81.95 92.88) (width 0.25) (layer "F.Cu") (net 2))
 (segment (start 81.32 92.25) (end 80.325 92.25) (width 0.25) (layer "F.Cu") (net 2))
 (segment (start 81.95 95) (end 81.95 94.35) (width 0.25) (layer "F.Cu") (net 2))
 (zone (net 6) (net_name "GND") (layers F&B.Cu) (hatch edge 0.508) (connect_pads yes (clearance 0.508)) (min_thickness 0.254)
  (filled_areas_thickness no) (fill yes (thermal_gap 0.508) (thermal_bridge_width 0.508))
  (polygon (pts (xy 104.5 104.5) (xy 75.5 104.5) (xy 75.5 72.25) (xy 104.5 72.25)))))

